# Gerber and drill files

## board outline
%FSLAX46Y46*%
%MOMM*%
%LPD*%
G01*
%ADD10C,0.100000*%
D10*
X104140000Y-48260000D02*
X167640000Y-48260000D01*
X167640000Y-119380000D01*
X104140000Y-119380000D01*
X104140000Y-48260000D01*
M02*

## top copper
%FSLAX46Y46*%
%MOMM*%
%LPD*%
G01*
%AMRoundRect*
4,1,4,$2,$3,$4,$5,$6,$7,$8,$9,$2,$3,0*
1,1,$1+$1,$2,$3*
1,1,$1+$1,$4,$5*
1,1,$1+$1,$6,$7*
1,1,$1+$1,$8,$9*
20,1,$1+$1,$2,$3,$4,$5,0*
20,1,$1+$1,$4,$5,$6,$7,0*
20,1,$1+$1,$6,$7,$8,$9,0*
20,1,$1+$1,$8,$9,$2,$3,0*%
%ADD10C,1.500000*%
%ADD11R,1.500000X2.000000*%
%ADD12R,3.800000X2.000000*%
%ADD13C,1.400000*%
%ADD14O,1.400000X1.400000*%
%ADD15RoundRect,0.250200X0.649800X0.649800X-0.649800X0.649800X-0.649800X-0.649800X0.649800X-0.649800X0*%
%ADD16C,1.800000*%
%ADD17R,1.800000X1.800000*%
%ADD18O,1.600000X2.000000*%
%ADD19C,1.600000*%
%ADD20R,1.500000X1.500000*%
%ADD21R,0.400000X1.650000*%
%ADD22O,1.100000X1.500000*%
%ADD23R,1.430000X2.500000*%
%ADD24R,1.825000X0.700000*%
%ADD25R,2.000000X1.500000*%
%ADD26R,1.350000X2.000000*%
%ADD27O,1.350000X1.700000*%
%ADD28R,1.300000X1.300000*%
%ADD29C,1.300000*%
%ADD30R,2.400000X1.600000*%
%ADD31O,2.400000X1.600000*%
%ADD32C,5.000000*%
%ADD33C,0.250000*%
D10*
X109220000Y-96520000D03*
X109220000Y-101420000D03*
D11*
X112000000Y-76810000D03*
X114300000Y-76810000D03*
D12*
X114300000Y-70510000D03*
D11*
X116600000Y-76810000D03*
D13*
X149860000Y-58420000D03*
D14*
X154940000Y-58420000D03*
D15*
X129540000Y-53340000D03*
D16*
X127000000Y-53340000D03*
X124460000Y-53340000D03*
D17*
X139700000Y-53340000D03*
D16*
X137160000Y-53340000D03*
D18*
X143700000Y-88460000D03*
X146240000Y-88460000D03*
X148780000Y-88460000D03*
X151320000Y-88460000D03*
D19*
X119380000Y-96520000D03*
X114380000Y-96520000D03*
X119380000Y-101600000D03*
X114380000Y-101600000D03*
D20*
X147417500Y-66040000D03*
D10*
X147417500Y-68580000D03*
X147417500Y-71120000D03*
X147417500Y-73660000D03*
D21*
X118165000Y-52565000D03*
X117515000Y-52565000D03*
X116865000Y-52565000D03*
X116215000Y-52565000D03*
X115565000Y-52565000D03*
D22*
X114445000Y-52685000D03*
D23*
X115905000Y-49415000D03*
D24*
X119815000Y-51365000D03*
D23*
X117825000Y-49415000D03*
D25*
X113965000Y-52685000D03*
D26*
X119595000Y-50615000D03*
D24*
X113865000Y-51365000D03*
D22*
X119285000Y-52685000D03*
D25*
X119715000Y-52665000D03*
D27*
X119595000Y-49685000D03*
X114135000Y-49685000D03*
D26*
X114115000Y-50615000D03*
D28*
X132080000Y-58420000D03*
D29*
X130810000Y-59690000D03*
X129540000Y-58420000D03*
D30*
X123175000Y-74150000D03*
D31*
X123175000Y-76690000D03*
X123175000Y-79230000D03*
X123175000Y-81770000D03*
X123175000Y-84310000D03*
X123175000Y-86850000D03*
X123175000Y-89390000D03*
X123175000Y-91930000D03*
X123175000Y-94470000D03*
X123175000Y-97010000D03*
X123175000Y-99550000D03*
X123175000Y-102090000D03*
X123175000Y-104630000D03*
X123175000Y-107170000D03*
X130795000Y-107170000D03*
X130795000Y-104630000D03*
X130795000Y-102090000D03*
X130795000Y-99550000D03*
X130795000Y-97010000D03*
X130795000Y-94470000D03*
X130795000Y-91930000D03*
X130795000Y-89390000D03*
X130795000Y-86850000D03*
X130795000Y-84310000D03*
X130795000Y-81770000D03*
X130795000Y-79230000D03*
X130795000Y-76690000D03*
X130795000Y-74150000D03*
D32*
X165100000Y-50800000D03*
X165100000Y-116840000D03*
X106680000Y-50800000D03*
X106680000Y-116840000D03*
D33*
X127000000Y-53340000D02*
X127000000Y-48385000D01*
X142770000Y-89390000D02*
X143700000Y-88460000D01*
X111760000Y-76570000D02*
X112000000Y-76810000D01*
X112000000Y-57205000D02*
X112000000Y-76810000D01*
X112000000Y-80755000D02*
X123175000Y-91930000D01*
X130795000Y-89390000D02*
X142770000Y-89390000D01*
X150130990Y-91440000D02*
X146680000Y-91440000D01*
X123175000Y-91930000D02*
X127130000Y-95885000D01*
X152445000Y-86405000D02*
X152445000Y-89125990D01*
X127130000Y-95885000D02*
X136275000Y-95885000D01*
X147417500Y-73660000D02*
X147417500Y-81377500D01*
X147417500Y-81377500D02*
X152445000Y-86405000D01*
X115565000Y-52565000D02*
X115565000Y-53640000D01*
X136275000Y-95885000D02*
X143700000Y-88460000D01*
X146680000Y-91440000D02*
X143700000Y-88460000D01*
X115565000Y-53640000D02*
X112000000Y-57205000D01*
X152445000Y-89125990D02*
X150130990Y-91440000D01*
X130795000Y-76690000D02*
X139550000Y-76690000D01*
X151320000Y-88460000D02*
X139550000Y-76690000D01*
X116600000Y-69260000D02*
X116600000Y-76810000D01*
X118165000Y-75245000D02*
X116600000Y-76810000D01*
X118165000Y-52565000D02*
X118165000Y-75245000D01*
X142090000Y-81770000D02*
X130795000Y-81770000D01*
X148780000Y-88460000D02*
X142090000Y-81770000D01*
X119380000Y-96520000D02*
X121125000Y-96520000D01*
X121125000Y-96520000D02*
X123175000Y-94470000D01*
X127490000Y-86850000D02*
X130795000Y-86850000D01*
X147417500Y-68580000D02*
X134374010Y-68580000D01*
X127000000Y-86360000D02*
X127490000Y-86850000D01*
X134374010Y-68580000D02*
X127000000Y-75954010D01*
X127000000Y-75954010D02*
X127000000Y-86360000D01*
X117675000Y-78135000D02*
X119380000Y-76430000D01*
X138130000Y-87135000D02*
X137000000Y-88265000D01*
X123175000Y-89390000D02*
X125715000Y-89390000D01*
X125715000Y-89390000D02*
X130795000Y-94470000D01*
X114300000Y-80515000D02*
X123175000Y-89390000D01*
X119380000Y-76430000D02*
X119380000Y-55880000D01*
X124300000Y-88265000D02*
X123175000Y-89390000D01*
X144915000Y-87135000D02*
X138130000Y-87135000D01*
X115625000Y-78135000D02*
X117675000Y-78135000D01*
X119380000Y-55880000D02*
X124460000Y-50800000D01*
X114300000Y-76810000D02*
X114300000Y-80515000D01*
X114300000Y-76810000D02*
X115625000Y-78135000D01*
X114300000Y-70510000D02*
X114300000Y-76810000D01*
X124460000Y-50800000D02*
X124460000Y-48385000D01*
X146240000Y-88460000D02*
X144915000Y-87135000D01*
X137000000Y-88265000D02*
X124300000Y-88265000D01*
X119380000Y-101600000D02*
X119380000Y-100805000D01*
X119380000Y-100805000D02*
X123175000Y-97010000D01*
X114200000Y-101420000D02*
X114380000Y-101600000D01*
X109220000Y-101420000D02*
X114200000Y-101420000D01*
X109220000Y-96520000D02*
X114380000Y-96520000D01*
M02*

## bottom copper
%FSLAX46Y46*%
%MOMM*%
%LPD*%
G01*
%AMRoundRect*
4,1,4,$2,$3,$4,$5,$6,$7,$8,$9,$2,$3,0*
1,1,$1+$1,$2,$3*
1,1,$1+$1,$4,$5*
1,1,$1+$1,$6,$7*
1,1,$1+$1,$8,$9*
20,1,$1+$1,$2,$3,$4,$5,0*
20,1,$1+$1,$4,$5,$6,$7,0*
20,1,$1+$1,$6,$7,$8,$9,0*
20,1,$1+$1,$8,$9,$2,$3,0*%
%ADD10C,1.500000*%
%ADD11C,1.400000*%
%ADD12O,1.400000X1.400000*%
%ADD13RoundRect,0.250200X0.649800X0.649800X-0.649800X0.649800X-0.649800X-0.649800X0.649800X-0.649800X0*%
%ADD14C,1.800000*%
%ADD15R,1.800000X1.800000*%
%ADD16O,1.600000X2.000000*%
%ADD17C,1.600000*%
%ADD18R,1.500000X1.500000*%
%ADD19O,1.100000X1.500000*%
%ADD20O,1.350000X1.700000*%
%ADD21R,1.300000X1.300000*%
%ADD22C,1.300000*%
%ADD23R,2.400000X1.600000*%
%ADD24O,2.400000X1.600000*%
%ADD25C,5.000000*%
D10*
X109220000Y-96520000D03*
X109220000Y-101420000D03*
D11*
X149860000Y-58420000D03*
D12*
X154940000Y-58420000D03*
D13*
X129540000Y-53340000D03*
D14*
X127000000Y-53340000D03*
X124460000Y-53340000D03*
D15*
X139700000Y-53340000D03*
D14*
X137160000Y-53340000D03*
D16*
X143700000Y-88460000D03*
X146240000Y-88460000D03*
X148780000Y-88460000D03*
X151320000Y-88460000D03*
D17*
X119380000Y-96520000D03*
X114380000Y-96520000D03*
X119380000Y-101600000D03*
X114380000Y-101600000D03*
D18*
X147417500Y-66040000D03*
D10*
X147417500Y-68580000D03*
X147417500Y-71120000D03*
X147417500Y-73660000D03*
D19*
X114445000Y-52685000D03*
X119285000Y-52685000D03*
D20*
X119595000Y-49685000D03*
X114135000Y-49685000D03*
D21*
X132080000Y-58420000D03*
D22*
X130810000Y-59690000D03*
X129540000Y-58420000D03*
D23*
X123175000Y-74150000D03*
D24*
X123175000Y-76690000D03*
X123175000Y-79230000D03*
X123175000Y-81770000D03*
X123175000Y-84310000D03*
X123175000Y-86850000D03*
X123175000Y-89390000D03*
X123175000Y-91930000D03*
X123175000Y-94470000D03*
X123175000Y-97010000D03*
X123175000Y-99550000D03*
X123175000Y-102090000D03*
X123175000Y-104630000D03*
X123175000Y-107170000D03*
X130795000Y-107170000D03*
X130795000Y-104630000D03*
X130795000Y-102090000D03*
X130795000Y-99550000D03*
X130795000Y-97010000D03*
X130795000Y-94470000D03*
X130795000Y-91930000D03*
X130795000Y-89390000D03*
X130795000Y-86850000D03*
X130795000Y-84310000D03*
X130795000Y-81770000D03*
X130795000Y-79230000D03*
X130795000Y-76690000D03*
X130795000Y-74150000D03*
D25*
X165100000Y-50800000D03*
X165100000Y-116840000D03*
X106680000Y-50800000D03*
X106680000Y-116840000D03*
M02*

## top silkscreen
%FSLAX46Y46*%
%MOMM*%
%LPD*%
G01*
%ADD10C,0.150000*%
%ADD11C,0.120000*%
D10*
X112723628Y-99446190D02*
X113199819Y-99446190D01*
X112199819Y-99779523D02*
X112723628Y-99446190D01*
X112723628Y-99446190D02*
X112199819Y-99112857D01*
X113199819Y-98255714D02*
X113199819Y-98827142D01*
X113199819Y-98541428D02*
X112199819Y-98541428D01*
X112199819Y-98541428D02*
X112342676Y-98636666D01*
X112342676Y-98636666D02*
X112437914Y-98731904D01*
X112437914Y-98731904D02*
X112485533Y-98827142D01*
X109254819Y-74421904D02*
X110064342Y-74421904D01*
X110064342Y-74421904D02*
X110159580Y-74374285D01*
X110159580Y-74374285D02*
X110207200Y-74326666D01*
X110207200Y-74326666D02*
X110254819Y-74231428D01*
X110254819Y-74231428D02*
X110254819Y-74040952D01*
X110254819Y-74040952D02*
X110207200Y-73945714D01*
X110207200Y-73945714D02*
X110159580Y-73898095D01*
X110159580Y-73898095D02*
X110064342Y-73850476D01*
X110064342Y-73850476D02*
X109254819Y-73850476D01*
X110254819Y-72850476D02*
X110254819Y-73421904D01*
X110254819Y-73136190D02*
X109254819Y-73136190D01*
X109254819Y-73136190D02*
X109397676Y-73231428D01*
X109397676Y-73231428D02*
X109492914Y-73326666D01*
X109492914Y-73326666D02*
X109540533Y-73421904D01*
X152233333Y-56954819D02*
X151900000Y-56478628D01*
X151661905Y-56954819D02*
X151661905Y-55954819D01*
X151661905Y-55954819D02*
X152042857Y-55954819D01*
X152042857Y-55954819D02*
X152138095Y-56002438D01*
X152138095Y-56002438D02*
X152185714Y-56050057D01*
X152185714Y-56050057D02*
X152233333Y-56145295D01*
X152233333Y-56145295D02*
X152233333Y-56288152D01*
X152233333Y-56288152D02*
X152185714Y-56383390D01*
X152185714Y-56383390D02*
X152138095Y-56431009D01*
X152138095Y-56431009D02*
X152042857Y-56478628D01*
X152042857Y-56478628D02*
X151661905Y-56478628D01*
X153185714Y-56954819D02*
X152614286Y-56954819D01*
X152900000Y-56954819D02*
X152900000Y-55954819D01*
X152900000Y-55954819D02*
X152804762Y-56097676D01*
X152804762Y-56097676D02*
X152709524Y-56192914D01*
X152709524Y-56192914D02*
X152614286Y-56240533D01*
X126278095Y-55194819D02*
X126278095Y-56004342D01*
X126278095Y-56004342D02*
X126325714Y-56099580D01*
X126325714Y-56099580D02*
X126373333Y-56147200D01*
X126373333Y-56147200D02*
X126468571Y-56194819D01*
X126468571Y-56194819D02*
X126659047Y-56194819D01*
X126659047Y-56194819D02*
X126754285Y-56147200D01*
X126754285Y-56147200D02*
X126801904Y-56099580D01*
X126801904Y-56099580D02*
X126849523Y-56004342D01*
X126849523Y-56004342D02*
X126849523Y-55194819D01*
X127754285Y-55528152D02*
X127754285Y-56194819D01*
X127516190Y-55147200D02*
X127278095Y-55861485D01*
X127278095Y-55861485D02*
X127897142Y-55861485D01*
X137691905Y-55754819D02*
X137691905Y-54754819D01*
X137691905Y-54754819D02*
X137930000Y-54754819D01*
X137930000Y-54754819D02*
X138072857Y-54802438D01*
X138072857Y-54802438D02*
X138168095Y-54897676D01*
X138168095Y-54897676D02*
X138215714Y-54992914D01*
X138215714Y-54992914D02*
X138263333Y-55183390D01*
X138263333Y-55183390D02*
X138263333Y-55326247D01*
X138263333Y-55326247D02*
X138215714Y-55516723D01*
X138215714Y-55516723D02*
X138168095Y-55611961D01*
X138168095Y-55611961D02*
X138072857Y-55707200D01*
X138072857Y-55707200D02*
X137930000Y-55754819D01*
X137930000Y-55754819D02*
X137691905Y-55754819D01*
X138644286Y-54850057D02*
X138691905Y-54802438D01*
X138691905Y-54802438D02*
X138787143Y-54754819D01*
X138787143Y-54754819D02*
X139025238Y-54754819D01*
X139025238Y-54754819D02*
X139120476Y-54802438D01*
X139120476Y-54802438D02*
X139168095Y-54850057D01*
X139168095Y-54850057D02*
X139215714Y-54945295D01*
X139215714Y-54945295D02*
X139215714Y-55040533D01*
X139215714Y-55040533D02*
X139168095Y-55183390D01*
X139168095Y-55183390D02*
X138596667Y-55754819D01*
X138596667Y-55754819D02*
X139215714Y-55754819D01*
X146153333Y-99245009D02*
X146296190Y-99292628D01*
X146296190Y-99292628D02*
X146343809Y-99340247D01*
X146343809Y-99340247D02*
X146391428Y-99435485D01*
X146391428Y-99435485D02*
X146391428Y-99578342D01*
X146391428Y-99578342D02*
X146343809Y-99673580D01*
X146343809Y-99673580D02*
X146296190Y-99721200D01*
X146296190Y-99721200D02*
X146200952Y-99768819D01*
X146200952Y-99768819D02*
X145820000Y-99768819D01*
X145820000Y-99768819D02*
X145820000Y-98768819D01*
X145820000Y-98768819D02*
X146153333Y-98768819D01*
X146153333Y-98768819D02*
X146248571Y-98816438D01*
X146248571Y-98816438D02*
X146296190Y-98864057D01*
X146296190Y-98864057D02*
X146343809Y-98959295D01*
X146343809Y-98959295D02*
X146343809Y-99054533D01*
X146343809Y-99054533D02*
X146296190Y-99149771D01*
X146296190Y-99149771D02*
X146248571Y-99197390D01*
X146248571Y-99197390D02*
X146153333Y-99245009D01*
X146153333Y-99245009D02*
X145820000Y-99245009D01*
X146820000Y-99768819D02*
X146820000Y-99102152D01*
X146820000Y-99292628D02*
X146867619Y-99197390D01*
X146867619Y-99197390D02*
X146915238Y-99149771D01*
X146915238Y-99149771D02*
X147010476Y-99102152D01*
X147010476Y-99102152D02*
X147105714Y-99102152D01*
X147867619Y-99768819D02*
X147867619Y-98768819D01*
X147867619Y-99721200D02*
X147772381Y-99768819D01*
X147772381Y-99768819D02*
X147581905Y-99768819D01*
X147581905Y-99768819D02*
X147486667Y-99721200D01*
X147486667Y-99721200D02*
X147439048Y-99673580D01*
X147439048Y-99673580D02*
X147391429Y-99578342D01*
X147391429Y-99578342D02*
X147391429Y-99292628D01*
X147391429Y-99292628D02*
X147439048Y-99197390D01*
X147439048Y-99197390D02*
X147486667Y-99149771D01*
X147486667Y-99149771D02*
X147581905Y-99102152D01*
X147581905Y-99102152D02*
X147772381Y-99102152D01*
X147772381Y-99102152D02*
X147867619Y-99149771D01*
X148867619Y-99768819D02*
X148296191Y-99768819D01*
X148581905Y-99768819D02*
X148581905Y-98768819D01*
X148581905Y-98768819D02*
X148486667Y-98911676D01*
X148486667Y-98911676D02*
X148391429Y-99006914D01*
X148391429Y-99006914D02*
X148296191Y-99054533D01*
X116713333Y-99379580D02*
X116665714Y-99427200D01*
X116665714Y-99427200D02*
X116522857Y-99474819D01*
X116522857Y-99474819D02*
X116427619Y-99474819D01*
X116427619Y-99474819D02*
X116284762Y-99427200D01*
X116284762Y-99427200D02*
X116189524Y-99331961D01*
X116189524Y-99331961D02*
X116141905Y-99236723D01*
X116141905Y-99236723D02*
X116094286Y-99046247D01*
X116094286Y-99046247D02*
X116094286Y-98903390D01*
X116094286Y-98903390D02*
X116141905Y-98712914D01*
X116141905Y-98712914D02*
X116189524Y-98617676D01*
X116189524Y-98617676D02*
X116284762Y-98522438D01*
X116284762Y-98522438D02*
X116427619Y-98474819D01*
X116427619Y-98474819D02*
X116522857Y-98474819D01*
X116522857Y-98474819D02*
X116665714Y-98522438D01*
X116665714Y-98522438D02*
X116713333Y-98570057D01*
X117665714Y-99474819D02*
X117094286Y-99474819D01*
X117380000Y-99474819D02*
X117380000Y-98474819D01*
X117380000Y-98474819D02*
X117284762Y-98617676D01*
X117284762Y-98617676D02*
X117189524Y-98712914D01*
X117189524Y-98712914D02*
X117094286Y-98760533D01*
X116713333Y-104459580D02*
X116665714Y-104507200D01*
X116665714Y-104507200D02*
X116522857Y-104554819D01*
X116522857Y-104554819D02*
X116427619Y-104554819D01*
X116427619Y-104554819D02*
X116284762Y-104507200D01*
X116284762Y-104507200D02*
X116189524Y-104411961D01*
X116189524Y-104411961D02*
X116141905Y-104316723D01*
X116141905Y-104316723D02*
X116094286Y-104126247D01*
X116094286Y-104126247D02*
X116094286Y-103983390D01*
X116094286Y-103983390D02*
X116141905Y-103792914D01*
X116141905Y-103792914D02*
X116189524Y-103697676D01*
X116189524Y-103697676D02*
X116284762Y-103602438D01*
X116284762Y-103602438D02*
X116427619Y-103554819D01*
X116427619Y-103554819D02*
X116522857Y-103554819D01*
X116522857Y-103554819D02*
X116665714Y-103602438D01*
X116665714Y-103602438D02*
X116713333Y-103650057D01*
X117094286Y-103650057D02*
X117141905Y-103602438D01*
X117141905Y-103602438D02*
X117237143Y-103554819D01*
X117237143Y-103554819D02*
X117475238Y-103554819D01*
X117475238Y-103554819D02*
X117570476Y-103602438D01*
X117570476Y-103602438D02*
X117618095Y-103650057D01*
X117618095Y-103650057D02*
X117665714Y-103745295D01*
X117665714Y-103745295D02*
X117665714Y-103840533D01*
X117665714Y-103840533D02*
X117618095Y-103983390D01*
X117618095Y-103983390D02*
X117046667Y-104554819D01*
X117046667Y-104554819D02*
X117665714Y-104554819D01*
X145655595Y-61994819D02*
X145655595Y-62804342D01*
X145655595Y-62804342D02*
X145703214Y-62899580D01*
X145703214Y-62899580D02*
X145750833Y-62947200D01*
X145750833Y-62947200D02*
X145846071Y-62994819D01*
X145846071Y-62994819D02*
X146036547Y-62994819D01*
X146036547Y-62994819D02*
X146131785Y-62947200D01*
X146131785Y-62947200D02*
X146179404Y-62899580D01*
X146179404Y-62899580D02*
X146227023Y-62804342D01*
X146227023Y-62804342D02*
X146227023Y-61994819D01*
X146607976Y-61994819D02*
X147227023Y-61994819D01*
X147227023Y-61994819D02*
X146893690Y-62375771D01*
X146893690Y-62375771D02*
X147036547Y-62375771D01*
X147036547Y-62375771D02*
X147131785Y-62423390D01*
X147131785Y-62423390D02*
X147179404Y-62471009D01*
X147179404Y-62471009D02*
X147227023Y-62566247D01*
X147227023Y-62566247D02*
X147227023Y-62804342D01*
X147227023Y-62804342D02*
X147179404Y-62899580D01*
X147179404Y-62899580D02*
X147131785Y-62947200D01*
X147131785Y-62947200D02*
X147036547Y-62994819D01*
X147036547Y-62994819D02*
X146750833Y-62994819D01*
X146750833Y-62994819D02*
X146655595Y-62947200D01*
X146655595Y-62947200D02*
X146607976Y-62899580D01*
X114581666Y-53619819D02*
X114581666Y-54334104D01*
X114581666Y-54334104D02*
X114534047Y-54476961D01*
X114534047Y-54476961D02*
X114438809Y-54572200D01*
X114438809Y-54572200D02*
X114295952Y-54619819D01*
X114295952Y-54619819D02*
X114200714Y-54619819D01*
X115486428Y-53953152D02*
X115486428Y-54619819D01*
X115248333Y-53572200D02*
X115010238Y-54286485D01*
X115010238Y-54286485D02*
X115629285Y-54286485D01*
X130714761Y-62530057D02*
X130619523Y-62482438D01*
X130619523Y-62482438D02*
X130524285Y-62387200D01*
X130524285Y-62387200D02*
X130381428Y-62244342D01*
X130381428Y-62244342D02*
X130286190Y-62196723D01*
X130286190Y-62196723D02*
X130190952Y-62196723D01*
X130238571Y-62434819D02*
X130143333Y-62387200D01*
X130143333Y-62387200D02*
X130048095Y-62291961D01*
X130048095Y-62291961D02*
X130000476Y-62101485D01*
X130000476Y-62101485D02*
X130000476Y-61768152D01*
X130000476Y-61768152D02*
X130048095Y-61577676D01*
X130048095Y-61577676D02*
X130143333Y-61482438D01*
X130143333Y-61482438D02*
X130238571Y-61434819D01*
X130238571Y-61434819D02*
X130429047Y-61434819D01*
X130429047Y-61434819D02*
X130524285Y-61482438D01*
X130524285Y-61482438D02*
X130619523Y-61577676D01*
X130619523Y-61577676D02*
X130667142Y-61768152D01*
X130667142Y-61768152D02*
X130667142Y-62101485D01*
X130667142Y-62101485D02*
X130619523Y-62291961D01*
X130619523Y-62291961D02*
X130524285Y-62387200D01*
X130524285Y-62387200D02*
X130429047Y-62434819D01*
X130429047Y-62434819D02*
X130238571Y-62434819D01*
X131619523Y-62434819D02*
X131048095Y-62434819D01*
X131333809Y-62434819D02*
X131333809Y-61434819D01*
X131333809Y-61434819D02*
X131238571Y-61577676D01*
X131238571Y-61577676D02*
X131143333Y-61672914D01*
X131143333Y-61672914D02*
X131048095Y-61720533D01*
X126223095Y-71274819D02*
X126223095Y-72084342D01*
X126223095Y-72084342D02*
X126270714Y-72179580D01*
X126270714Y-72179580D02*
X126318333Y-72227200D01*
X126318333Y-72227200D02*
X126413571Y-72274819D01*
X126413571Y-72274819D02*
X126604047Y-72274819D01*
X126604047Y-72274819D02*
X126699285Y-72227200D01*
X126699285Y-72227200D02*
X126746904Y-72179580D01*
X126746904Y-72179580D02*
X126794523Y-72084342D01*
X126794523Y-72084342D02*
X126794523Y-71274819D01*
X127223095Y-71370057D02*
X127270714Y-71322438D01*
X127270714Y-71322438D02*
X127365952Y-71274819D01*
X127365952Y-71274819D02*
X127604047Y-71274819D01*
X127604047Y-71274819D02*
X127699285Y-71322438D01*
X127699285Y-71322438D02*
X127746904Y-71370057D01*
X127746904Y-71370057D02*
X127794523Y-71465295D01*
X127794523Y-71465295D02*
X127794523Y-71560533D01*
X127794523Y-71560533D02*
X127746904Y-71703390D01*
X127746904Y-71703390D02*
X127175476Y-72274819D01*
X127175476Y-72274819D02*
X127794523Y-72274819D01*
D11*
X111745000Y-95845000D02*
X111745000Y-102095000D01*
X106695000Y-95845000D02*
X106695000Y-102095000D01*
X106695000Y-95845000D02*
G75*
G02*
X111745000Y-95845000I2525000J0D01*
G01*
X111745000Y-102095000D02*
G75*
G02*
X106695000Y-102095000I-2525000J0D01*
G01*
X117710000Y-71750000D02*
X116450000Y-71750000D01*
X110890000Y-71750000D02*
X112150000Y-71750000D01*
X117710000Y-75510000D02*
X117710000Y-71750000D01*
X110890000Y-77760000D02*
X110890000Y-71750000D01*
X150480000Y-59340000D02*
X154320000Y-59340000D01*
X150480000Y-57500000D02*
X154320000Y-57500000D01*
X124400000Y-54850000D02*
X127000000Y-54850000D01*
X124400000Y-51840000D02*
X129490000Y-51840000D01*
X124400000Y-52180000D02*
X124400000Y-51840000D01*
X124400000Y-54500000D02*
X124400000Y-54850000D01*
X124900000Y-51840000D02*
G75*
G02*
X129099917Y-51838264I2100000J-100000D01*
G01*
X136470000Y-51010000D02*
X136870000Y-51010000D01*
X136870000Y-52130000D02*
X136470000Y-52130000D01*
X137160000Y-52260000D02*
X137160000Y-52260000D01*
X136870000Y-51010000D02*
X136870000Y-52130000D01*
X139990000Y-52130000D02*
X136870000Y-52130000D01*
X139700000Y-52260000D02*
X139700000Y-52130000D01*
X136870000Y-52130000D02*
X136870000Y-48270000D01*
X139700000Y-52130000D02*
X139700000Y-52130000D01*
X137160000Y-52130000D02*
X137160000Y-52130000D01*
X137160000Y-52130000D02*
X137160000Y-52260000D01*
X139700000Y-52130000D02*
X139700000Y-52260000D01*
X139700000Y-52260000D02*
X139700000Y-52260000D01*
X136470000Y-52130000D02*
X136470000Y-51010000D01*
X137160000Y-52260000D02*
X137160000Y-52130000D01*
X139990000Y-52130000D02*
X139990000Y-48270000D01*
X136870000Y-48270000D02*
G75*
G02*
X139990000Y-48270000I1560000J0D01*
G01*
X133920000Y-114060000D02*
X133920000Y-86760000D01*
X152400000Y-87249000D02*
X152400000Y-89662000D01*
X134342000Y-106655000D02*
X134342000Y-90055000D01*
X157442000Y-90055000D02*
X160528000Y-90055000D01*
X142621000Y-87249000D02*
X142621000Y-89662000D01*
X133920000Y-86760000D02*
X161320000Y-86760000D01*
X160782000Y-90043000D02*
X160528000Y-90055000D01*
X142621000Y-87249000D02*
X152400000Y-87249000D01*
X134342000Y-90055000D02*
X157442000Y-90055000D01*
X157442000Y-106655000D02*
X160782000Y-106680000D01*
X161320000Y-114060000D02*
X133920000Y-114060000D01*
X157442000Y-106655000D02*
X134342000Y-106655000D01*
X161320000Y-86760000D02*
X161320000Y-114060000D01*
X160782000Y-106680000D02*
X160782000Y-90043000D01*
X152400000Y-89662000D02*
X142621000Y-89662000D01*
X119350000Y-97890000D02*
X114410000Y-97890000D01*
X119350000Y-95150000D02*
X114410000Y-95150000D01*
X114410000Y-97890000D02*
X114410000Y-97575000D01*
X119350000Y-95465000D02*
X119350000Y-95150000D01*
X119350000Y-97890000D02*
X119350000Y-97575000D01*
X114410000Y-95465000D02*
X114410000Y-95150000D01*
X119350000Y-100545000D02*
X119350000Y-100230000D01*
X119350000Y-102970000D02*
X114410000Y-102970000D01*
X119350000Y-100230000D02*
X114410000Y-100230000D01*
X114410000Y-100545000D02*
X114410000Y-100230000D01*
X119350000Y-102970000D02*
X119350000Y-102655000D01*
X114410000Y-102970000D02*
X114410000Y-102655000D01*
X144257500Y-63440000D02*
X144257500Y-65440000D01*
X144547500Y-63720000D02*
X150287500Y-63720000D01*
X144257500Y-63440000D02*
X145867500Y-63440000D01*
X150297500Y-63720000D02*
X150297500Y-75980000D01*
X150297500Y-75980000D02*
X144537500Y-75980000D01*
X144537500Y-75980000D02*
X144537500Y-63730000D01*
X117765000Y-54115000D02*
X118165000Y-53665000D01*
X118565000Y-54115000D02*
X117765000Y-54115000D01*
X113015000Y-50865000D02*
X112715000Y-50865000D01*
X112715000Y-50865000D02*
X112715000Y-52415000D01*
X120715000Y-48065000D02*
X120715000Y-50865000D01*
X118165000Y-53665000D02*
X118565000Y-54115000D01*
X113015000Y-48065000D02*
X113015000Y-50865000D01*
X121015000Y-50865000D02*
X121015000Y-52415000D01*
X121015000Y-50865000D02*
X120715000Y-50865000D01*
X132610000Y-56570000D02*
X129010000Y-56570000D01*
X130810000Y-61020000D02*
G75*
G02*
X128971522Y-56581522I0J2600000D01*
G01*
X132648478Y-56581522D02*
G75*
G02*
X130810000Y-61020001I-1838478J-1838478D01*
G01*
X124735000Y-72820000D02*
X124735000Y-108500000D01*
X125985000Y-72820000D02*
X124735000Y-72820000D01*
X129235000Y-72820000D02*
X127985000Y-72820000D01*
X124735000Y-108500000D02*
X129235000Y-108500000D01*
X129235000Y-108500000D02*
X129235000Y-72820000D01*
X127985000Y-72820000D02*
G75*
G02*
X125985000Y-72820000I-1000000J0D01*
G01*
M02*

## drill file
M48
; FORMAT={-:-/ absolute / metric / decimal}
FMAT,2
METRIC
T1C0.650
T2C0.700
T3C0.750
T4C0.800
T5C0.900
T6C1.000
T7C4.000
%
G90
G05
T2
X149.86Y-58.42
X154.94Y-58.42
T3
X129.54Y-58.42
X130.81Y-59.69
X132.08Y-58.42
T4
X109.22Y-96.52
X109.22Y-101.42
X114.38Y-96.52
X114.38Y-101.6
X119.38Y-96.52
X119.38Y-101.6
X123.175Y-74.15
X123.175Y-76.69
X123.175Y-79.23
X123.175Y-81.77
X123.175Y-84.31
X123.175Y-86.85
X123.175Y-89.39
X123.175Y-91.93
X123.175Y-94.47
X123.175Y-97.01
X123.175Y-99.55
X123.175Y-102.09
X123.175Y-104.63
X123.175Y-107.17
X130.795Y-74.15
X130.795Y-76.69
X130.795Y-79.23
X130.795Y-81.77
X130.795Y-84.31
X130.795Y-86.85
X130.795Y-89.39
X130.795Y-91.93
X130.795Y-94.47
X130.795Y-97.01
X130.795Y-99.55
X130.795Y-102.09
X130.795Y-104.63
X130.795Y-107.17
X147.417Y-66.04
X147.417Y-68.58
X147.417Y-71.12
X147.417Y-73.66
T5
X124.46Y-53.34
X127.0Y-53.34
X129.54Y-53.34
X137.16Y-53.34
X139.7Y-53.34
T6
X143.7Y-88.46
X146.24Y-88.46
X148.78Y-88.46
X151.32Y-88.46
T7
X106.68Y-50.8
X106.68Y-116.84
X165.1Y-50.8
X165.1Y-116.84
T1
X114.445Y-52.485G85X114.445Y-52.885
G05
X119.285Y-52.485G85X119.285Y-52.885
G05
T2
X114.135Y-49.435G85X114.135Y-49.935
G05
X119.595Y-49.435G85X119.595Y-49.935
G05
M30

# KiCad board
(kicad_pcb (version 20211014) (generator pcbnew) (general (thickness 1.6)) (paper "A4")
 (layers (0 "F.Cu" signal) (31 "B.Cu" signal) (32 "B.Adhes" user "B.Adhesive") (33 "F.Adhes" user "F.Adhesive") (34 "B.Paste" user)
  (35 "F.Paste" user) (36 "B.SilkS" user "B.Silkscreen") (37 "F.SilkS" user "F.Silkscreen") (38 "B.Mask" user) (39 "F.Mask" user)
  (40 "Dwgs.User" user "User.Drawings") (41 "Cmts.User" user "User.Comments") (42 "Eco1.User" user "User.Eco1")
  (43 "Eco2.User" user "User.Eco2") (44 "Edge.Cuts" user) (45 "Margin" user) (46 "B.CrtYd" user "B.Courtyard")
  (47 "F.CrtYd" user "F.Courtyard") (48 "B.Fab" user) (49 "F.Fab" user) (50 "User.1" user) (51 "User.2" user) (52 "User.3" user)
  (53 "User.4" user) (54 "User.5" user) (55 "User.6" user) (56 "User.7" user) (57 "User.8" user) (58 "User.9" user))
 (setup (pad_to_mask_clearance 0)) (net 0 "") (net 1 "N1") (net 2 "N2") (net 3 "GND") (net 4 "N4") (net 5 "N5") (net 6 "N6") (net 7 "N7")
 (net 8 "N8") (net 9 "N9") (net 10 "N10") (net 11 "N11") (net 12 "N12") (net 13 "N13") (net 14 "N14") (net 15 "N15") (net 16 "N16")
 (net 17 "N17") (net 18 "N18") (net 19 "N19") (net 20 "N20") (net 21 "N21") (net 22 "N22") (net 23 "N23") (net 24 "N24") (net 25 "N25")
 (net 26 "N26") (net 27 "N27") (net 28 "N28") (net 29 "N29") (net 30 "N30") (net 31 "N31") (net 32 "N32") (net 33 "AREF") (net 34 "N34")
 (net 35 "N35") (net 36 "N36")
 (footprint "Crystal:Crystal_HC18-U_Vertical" (layer "F.Cu") (at 109.22 96.52 -90)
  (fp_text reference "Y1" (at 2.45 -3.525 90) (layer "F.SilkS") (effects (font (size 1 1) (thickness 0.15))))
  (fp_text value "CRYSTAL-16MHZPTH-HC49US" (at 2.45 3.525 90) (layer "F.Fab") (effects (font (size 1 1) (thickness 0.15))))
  (fp_line (start -0.675 -2.525) (end 5.575 -2.525) (layer "F.SilkS") (width 0.12))
  (fp_line (start -0.675 2.525) (end 5.575 2.525) (layer "F.SilkS") (width 0.12))
  (fp_arc (start -0.675 2.525) (mid -3.2 0) (end -0.675 -2.525) (layer "F.SilkS") (width 0.12))
  (fp_arc (start 5.575 -2.525) (mid 8.1 0) (end 5.575 2.525) (layer "F.SilkS") (width 0.12))
  (pad "1" thru_hole circle (at 0 0 270) (size 1.5 1.5) (drill 0.8) (layers *.Cu *.Mask) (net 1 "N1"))
  (pad "2" thru_hole circle (at 4.9 0 270) (size 1.5 1.5) (drill 0.8) (layers *.Cu *.Mask) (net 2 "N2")))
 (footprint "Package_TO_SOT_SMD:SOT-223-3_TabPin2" (layer "F.Cu") (at 114.3 73.66 90)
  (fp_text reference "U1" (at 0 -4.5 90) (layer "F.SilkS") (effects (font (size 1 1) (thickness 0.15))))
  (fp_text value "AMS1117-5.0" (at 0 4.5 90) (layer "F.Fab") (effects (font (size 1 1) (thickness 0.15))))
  (fp_line (start 1.91 3.41) (end 1.91 2.15) (layer "F.SilkS") (width 0.12))
  (fp_line (start 1.91 -3.41) (end 1.91 -2.15) (layer "F.SilkS") (width 0.12))
  (fp_line (start -1.85 3.41) (end 1.91 3.41) (layer "F.SilkS") (width 0.12))
  (fp_line (start -4.1 -3.41) (end 1.91 -3.41) (layer "F.SilkS") (width 0.12))
  (pad "1" smd rect (at -3.15 -2.3 90) (size 2 1.5) (layers "F.Cu" "F.Paste" "F.Mask") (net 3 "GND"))
  (pad "2" smd rect (at -3.15 0 90) (size 2 1.5) (layers "F.Cu" "F.Paste" "F.Mask") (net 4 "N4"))
  (pad "2" smd rect (at 3.15 0 90) (size 2 3.8) (layers "F.Cu" "F.Paste" "F.Mask") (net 4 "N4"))
  (pad "3" smd rect (at -3.15 2.3 90) (size 2 1.5) (layers "F.Cu" "F.Paste" "F.Mask") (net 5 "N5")))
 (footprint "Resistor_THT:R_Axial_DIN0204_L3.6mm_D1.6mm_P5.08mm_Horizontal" (layer "F.Cu") (at 149.86 58.42)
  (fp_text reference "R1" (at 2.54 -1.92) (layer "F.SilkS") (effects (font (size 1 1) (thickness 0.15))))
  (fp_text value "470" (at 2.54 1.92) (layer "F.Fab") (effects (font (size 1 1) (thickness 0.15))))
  (fp_line (start 0.62 0.92) (end 4.46 0.92) (layer "F.SilkS") (width 0.12))
  (fp_line (start 0.62 -0.92) (end 4.46 -0.92) (layer "F.SilkS") (width 0.12))
  (pad "1" thru_hole circle (at 0 0) (size 1.4 1.4) (drill 0.7) (layers *.Cu *.Mask) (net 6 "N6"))
  (pad "2" thru_hole oval (at 5.08 0) (size 1.4 1.4) (drill 0.7) (layers *.Cu *.Mask) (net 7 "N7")))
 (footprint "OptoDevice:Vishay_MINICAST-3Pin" (layer "F.Cu") (at 129.54 53.34 180)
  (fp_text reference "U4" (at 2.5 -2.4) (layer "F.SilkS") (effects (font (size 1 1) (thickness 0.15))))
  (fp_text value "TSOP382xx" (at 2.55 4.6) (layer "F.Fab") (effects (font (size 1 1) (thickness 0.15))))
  (fp_line (start 5.14 -1.51) (end 2.54 -1.51) (layer "F.SilkS") (width 0.12))
  (fp_line (start 5.14 1.5) (end 0.05 1.5) (layer "F.SilkS") (width 0.12))
  (fp_line (start 5.14 1.16) (end 5.14 1.5) (layer "F.SilkS") (width 0.12))
  (fp_line (start 5.14 -1.16) (end 5.14 -1.51) (layer "F.SilkS") (width 0.12))
  (fp_arc (start 4.64 1.5) (mid 2.540869 3.502379) (end 0.440083 1.501736) (layer "F.SilkS") (width 0.12))
  (pad "1" thru_hole roundrect (at 0 0 180) (size 1.8 1.8) (drill 0.9) (layers *.Cu *.Mask) (roundrect_rratio 0.139) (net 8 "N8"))
  (pad "2" thru_hole circle (at 2.54 0 180) (size 1.8 1.8) (drill 0.9) (layers *.Cu *.Mask) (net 3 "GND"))
  (pad "3" thru_hole circle (at 5.08 0 180) (size 1.8 1.8) (drill 0.9) (layers *.Cu *.Mask) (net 4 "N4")))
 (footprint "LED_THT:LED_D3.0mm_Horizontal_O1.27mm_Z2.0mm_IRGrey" (layer "F.Cu") (at 139.7 53.34 180)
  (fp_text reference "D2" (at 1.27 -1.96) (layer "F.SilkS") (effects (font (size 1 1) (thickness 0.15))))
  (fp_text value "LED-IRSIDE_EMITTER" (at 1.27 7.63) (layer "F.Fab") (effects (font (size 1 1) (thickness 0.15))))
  (fp_line (start 3.23 2.33) (end 2.83 2.33) (layer "F.SilkS") (width 0.12))
  (fp_line (start 2.83 1.21) (end 3.23 1.21) (layer "F.SilkS") (width 0.12))
  (fp_line (start 2.54 1.08) (end 2.54 1.08) (layer "F.SilkS") (width 0.12))
  (fp_line (start 2.83 2.33) (end 2.83 1.21) (layer "F.SilkS") (width 0.12))
  (fp_line (start -0.29 1.21) (end 2.83 1.21) (layer "F.SilkS") (width 0.12))
  (fp_line (start 0 1.08) (end 0 1.21) (layer "F.SilkS") (width 0.12))
  (fp_line (start 2.83 1.21) (end 2.83 5.07) (layer "F.SilkS") (width 0.12))
  (fp_line (start 0 1.21) (end 0 1.21) (layer "F.SilkS") (width 0.12))
  (fp_line (start 2.54 1.21) (end 2.54 1.21) (layer "F.SilkS") (width 0.12))
  (fp_line (start 2.54 1.21) (end 2.54 1.08) (layer "F.SilkS") (width 0.12))
  (fp_line (start 0 1.21) (end 0 1.08) (layer "F.SilkS") (width 0.12))
  (fp_line (start 0 1.08) (end 0 1.08) (layer "F.SilkS") (width 0.12))
  (fp_line (start 3.23 1.21) (end 3.23 2.33) (layer "F.SilkS") (width 0.12))
  (fp_line (start 2.54 1.08) (end 2.54 1.21) (layer "F.SilkS") (width 0.12))
  (fp_line (start -0.29 1.21) (end -0.29 5.07) (layer "F.SilkS") (width 0.12))
  (fp_arc (start 2.83 5.07) (mid 1.27 6.63) (end -0.29 5.07) (layer "F.SilkS") (width 0.12))
  (pad "1" thru_hole rect (at 0 0 180) (size 1.8 1.8) (drill 0.9) (layers *.Cu *.Mask))
  (pad "2" thru_hole circle (at 2.54 0 180) (size 1.8 1.8) (drill 0.9) (layers *.Cu *.Mask)))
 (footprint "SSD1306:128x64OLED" (layer "F.Cu") (at 147.32 99.06)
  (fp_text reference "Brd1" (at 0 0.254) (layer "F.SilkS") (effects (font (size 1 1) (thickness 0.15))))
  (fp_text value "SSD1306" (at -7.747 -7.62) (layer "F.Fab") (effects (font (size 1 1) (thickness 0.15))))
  (fp_line (start -13.4 15) (end -13.4 -12.3) (layer "F.SilkS") (width 0.12))
  (fp_line (start 5.08 -11.811) (end 5.08 -9.398) (layer "F.SilkS") (width 0.12))
  (fp_line (start -12.978 7.595) (end -12.978 -9.005) (layer "F.SilkS") (width 0.12))
  (fp_line (start 10.122 -9.005) (end 13.208 -9.005) (layer "F.SilkS") (width 0.12))
  (fp_line (start -4.699 -11.811) (end -4.699 -9.398) (layer "F.SilkS") (width 0.12))
  (fp_line (start -13.4 -12.3) (end 14 -12.3) (layer "F.SilkS") (width 0.12))
  (fp_line (start 13.462 -9.017) (end 13.208 -9.005) (layer "F.SilkS") (width 0.12))
  (fp_line (start -4.699 -11.811) (end 5.08 -11.811) (layer "F.SilkS") (width 0.12))
  (fp_line (start -12.978 -9.005) (end 10.122 -9.005) (layer "F.SilkS") (width 0.12))
  (fp_line (start 10.122 7.595) (end 13.462 7.62) (layer "F.SilkS") (width 0.12))
  (fp_line (start 14 15) (end -13.4 15) (layer "F.SilkS") (width 0.12))
  (fp_line (start 10.122 7.595) (end -12.978 7.595) (layer "F.SilkS") (width 0.12))
  (fp_line (start 14 -12.3) (end 14 15) (layer "F.SilkS") (width 0.12))
  (fp_line (start 13.462 7.62) (end 13.462 -9.017) (layer "F.SilkS") (width 0.12))
  (fp_line (start 5.08 -9.398) (end -4.699 -9.398) (layer "F.SilkS") (width 0.12))
  (pad "1" thru_hole oval locked (at -3.62 -10.6 90) (size 2 1.6) (drill 1) (layers *.Cu *.Mask) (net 3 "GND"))
  (pad "2" thru_hole oval locked (at -1.08 -10.6 90) (size 2 1.6) (drill 1) (layers *.Cu *.Mask) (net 4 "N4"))
  (pad "3" thru_hole oval locked (at 1.46 -10.6 90) (size 2 1.6) (drill 1) (layers *.Cu *.Mask) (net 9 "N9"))
  (pad "4" thru_hole oval locked (at 4 -10.6 90) (size 2 1.6) (drill 1) (layers *.Cu *.Mask) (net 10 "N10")))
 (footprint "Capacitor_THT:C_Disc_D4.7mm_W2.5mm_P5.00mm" (layer "F.Cu") (at 119.38 96.52 180)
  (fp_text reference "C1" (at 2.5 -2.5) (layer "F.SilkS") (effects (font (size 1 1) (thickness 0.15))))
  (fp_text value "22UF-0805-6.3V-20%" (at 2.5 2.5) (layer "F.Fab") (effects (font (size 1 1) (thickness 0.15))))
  (fp_line (start 0.03 -1.37) (end 4.97 -1.37) (layer "F.SilkS") (width 0.12))
  (fp_line (start 0.03 1.37) (end 4.97 1.37) (layer "F.SilkS") (width 0.12))
  (fp_line (start 4.97 -1.37) (end 4.97 -1.055) (layer "F.SilkS") (width 0.12))
  (fp_line (start 0.03 1.055) (end 0.03 1.37) (layer "F.SilkS") (width 0.12))
  (fp_line (start 0.03 -1.37) (end 0.03 -1.055) (layer "F.SilkS") (width 0.12))
  (fp_line (start 4.97 1.055) (end 4.97 1.37) (layer "F.SilkS") (width 0.12))
  (pad "1" thru_hole circle (at 0 0 180) (size 1.6 1.6) (drill 0.8) (layers *.Cu *.Mask) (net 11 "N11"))
  (pad "2" thru_hole circle (at 5 0 180) (size 1.6 1.6) (drill 0.8) (layers *.Cu *.Mask) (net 1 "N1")))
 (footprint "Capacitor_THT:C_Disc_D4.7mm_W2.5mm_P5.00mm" (layer "F.Cu") (at 119.38 101.6 180)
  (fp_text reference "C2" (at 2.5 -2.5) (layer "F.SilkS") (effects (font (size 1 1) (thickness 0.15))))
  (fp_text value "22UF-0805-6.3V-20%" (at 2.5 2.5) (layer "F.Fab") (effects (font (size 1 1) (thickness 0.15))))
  (fp_line (start 0.03 1.055) (end 0.03 1.37) (layer "F.SilkS") (width 0.12))
  (fp_line (start 0.03 -1.37) (end 4.97 -1.37) (layer "F.SilkS") (width 0.12))
  (fp_line (start 0.03 1.37) (end 4.97 1.37) (layer "F.SilkS") (width 0.12))
  (fp_line (start 4.97 1.055) (end 4.97 1.37) (layer "F.SilkS") (width 0.12))
  (fp_line (start 0.03 -1.37) (end 0.03 -1.055) (layer "F.SilkS") (width 0.12))
  (fp_line (start 4.97 -1.37) (end 4.97 -1.055) (layer "F.SilkS") (width 0.12))
  (pad "1" thru_hole circle (at 0 0 180) (size 1.6 1.6) (drill 0.8) (layers *.Cu *.Mask) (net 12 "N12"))
  (pad "2" thru_hole circle (at 5 0 180) (size 1.6 1.6) (drill 0.8) (layers *.Cu *.Mask) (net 2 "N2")))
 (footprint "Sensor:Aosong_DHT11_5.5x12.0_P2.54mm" (layer "F.Cu") (at 147.4175 66.04)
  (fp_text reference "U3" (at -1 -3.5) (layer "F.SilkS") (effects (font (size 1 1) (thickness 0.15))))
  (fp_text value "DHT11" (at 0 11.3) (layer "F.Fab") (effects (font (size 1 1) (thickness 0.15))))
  (fp_line (start -3.16 -2.6) (end -3.16 -0.6) (layer "F.SilkS") (width 0.12))
  (fp_line (start -2.87 -2.32) (end 2.87 -2.32) (layer "F.SilkS") (width 0.12))
  (fp_line (start -3.16 -2.6) (end -1.55 -2.6) (layer "F.SilkS") (width 0.12))
  (fp_line (start 2.88 -2.32) (end 2.88 9.94) (layer "F.SilkS") (width 0.12))
  (fp_line (start 2.88 9.94) (end -2.88 9.94) (layer "F.SilkS") (width 0.12))
  (fp_line (start -2.88 9.94) (end -2.88 -2.31) (layer "F.SilkS") (width 0.12))
  (pad "1" thru_hole rect (at 0 0) (size 1.5 1.5) (drill 0.8) (layers *.Cu *.Mask) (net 4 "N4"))
  (pad "2" thru_hole circle (at 0 2.54) (size 1.5 1.5) (drill 0.8) (layers *.Cu *.Mask) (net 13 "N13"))
  (pad "3" thru_hole circle (at 0 5.08) (size 1.5 1.5) (drill 0.8) (layers *.Cu *.Mask) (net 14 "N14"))
  (pad "4" thru_hole circle (at 0 7.62) (size 1.5 1.5) (drill 0.8) (layers *.Cu *.Mask) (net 3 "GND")))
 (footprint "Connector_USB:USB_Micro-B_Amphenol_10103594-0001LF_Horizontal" (layer "F.Cu") (at 116.84 50.8 180)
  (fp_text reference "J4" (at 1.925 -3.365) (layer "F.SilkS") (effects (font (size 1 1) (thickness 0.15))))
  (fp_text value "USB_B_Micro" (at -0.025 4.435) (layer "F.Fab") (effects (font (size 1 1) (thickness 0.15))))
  (fp_line (start -0.925 -3.315) (end -1.325 -2.865) (layer "F.SilkS") (width 0.12))
  (fp_line (start -1.725 -3.315) (end -0.925 -3.315) (layer "F.SilkS") (width 0.12))
  (fp_line (start 3.825 -0.065) (end 4.125 -0.065) (layer "F.SilkS") (width 0.12))
  (fp_line (start 4.125 -0.065) (end 4.125 -1.615) (layer "F.SilkS") (width 0.12))
  (fp_line (start -3.875 2.735) (end -3.875 -0.065) (layer "F.SilkS") (width 0.12))
  (fp_line (start -1.325 -2.865) (end -1.725 -3.315) (layer "F.SilkS") (width 0.12))
  (fp_line (start 3.825 2.735) (end 3.825 -0.065) (layer "F.SilkS") (width 0.12))
  (fp_line (start -4.175 -0.065) (end -4.175 -1.615) (layer "F.SilkS") (width 0.12))
  (fp_line (start -4.175 -0.065) (end -3.875 -0.065) (layer "F.SilkS") (width 0.12))
  (pad "1" smd rect (at -1.325 -1.765 270) (size 1.65 0.4) (layers "F.Cu" "F.Paste" "F.Mask") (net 5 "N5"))
  (pad "2" smd rect (at -0.675 -1.765 270) (size 1.65 0.4) (layers "F.Cu" "F.Paste" "F.Mask") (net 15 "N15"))
  (pad "3" smd rect (at -0.025 -1.765 270) (size 1.65 0.4) (layers "F.Cu" "F.Paste" "F.Mask") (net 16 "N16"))
  (pad "4" smd rect (at 0.625 -1.765 270) (size 1.65 0.4) (layers "F.Cu" "F.Paste" "F.Mask") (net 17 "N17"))
  (pad "5" smd rect (at 1.275 -1.765 270) (size 1.65 0.4) (layers "F.Cu" "F.Paste" "F.Mask") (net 3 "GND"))
  (pad "6" thru_hole oval (at 2.395 -1.885 270) (size 1.5 1.1) (drill oval 1.05 0.65) (layers *.Cu *.Mask) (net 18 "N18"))
  (pad "6" smd rect (at 0.935 1.385 270) (size 2.5 1.43) (layers "F.Cu" "F.Paste" "F.Mask") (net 18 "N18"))
  (pad "6" smd rect (at -2.975 -0.565 180) (size 1.825 0.7) (layers "F.Cu" "F.Paste" "F.Mask") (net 18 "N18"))
  (pad "6" smd rect (at -0.985 1.385 270) (size 2.5 1.43) (layers "F.Cu" "F.Paste" "F.Mask") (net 18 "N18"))
  (pad "6" smd rect (at 2.875 -1.885 180) (size 2 1.5) (layers "F.Cu" "F.Paste" "F.Mask") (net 18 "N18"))
  (pad "6" smd rect (at -2.755 0.185 180) (size 1.35 2) (layers "F.Cu" "F.Paste" "F.Mask") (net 18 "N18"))
  (pad "6" smd rect (at 2.975 -0.565 180) (size 1.825 0.7) (layers "F.Cu" "F.Paste" "F.Mask") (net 18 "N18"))
  (pad "6" thru_hole oval (at -2.445 -1.885 270) (size 1.5 1.1) (drill oval 1.05 0.65) (layers *.Cu *.Mask) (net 18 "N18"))
  (pad "6" smd rect (at -2.875 -1.865 180) (size 2 1.5) (layers "F.Cu" "F.Paste" "F.Mask") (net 18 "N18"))
  (pad "6" thru_hole oval (at -2.755 1.115 270) (size 1.7 1.35) (drill oval 1.2 0.7) (layers *.Cu *.Mask) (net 18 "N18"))
  (pad "6" thru_hole oval (at 2.705 1.115 270) (size 1.7 1.35) (drill oval 1.2 0.7) (layers *.Cu *.Mask) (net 18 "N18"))
  (pad "6" smd rect (at 2.725 0.185 180) (size 1.35 2) (layers "F.Cu" "F.Paste" "F.Mask") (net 18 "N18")))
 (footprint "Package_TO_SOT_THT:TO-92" (layer "F.Cu") (at 132.08 58.42 180)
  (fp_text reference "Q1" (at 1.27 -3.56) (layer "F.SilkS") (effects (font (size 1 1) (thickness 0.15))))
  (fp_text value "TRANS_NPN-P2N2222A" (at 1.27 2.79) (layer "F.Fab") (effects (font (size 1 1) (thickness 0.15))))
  (fp_line (start -0.53 1.85) (end 3.07 1.85) (layer "F.SilkS") (width 0.12))
  (fp_arc (start 1.27 -2.6) (mid 3.672087 -0.994977) (end 3.108478 1.838478) (layer "F.SilkS") (width 0.12))
  (fp_arc (start -0.568478 1.838478) (mid -1.132087 -0.994977) (end 1.27 -2.6) (layer "F.SilkS") (width 0.12))
  (pad "1" thru_hole rect (at 0 0 180) (size 1.3 1.3) (drill 0.75) (layers *.Cu *.Mask) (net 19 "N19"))
  (pad "2" thru_hole circle (at 1.27 -1.27 180) (size 1.3 1.3) (drill 0.75) (layers *.Cu *.Mask) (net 7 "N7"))
  (pad "3" thru_hole circle (at 2.54 0 180) (size 1.3 1.3) (drill 0.75) (layers *.Cu *.Mask) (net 3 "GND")))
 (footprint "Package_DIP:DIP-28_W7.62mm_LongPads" (layer "F.Cu") (at 123.175 74.15)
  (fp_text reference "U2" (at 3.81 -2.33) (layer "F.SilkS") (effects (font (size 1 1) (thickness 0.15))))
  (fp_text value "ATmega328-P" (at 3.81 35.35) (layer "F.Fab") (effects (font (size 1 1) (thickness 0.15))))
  (fp_line (start 1.56 -1.33) (end 1.56 34.35) (layer "F.SilkS") (width 0.12))
  (fp_line (start 2.81 -1.33) (end 1.56 -1.33) (layer "F.SilkS") (width 0.12))
  (fp_line (start 6.06 -1.33) (end 4.81 -1.33) (layer "F.SilkS") (width 0.12))
  (fp_line (start 1.56 34.35) (end 6.06 34.35) (layer "F.SilkS") (width 0.12))
  (fp_line (start 6.06 34.35) (end 6.06 -1.33) (layer "F.SilkS") (width 0.12))
  (fp_arc (start 4.81 -1.33) (mid 3.81 -0.33) (end 2.81 -1.33) (layer "F.SilkS") (width 0.12))
  (pad "1" thru_hole rect (at 0 0) (size 2.4 1.6) (drill 0.8) (layers *.Cu *.Mask) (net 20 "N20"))
  (pad "2" thru_hole oval (at 0 2.54) (size 2.4 1.6) (drill 0.8) (layers *.Cu *.Mask) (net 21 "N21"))
  (pad "3" thru_hole oval (at 0 5.08) (size 2.4 1.6) (drill 0.8) (layers *.Cu *.Mask) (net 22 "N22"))
  (pad "4" thru_hole oval (at 0 7.62) (size 2.4 1.6) (drill 0.8) (layers *.Cu *.Mask) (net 6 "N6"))
  (pad "5" thru_hole oval (at 0 10.16) (size 2.4 1.6) (drill 0.8) (layers *.Cu *.Mask) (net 8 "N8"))
  (pad "6" thru_hole oval (at 0 12.7) (size 2.4 1.6) (drill 0.8) (layers *.Cu *.Mask) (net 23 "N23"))
  (pad "7" thru_hole oval (at 0 15.24) (size 2.4 1.6) (drill 0.8) (layers *.Cu *.Mask) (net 4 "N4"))
  (pad "8" thru_hole oval (at 0 17.78) (size 2.4 1.6) (drill 0.8) (layers *.Cu *.Mask) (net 3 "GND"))
  (pad "9" thru_hole oval (at 0 20.32) (size 2.4 1.6) (drill 0.8) (layers *.Cu *.Mask) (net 11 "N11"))
  (pad "10" thru_hole oval (at 0 22.86) (size 2.4 1.6) (drill 0.8) (layers *.Cu *.Mask) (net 12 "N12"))
  (pad "11" thru_hole oval (at 0 25.4) (size 2.4 1.6) (drill 0.8) (layers *.Cu *.Mask) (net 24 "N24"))
  (pad "12" thru_hole oval (at 0 27.94) (size 2.4 1.6) (drill 0.8) (layers *.Cu *.Mask) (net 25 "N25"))
  (pad "13" thru_hole oval (at 0 30.48) (size 2.4 1.6) (drill 0.8) (layers *.Cu *.Mask) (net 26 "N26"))
  (pad "14" thru_hole oval (at 0 33.02) (size 2.4 1.6) (drill 0.8) (layers *.Cu *.Mask) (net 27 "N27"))
  (pad "15" thru_hole oval (at 7.62 33.02) (size 2.4 1.6) (drill 0.8) (layers *.Cu *.Mask) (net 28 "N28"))
  (pad "16" thru_hole oval (at 7.62 30.48) (size 2.4 1.6) (drill 0.8) (layers *.Cu *.Mask) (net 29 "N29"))
  (pad "17" thru_hole oval (at 7.62 27.94) (size 2.4 1.6) (drill 0.8) (layers *.Cu *.Mask) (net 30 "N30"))
  (pad "18" thru_hole oval (at 7.62 25.4) (size 2.4 1.6) (drill 0.8) (layers *.Cu *.Mask) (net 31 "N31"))
  (pad "19" thru_hole oval (at 7.62 22.86) (size 2.4 1.6) (drill 0.8) (layers *.Cu *.Mask) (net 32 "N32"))
  (pad "20" thru_hole oval (at 7.62 20.32) (size 2.4 1.6) (drill 0.8) (layers *.Cu *.Mask) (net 4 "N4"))
  (pad "21" thru_hole oval (at 7.62 17.78) (size 2.4 1.6) (drill 0.8) (layers *.Cu *.Mask) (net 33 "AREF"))
  (pad "22" thru_hole oval (at 7.62 15.24) (size 2.4 1.6) (drill 0.8) (layers *.Cu *.Mask) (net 3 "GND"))
  (pad "23" thru_hole oval (at 7.62 12.7) (size 2.4 1.6) (drill 0.8) (layers *.Cu *.Mask) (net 13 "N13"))
  (pad "24" thru_hole oval (at 7.62 10.16) (size 2.4 1.6) (drill 0.8) (layers *.Cu *.Mask) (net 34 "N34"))
  (pad "25" thru_hole oval (at 7.62 7.62) (size 2.4 1.6) (drill 0.8) (layers *.Cu *.Mask) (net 9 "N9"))
  (pad "26" thru_hole oval (at 7.62 5.08) (size 2.4 1.6) (drill 0.8) (layers *.Cu *.Mask) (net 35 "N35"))
  (pad "27" thru_hole oval (at 7.62 2.54) (size 2.4 1.6) (drill 0.8) (layers *.Cu *.Mask) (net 10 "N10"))
  (pad "28" thru_hole oval (at 7.62 0) (size 2.4 1.6) (drill 0.8) (layers *.Cu *.Mask) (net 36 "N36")))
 (gr_rect (start 104.14 48.26) (end 167.64 119.38) (layer "Edge.Cuts") (width 0.1) (fill none))
 (via (at 165.1 50.8) (size 5) (drill 4) (layers "F.Cu" "B.Cu") (free) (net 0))
 (via (at 165.1 116.84) (size 5) (drill 4) (layers "F.Cu" "B.Cu") (free) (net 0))
 (via (at 106.68 50.8) (size 5) (drill 4) (layers "F.Cu" "B.Cu") (free) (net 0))
 (via (at 106.68 116.84) (size 5) (drill 4) (layers "F.Cu" "B.Cu") (free) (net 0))
 (segment (start 127 53.34) (end 127 48.385) (width 0.25) (layer "F.Cu") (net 3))
 (segment (start 142.77 89.39) (end 143.7 88.46) (width 0.25) (layer "F.Cu") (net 3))
 (segment (start 111.76 76.57) (end 112 76.81) (width 0.25) (layer "F.Cu") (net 3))
 (segment (start 112 57.205) (end 112 76.81) (width 0.25) (layer "F.Cu") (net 3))
 (segment (start 112 80.755) (end 123.175 91.93) (width 0.25) (layer "F.Cu") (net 3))
 (segment (start 130.795 89.39) (end 142.77 89.39) (width 0.25) (layer "F.Cu") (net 3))
 (segment (start 150.13099 91.44) (end 146.68 91.44) (width 0.25) (layer "F.Cu") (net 3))
 (segment (start 123.175 91.93) (end 127.13 95.885) (width 0.25) (layer "F.Cu") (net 3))
 (segment (start 152.445 86.405) (end 152.445 89.12599) (width 0.25) (layer "F.Cu") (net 3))
 (segment (start 127.13 95.885) (end 136.275 95.885) (width 0.25) (layer "F.Cu") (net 3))
 (segment (start 147.4175 73.66) (end 147.4175 81.3775) (width 0.25) (layer "F.Cu") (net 3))
 (segment (start 147.4175 81.3775) (end 152.445 86.405) (width 0.25) (layer "F.Cu") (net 3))
 (segment (start 115.565 52.565) (end 115.565 53.64) (width 0.25) (layer "F.Cu") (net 3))
 (segment (start 136.275 95.885) (end 143.7 88.46) (width 0.25) (layer "F.Cu") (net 3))
 (segment (start 146.68 91.44) (end 143.7 88.46) (width 0.25) (layer "F.Cu") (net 3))
 (segment (start 115.565 53.64) (end 112 57.205) (width 0.25) (layer "F.Cu") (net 3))
 (segment (start 152.445 89.12599) (end 150.13099 91.44) (width 0.25) (layer "F.Cu") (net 3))
 (segment (start 130.795 76.69) (end 139.55 76.69) (width 0.25) (layer "F.Cu") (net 10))
 (segment (start 151.32 88.46) (end 139.55 76.69) (width 0.25) (layer "F.Cu") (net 10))
 (segment (start 116.6 69.26) (end 116.6 76.81) (width 0.25) (layer "F.Cu") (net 5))
 (segment (start 118.165 75.245) (end 116.6 76.81) (width 0.25) (layer "F.Cu") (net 5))
 (segment (start 118.165 52.565) (end 118.165 75.245) (width 0.25) (layer "F.Cu") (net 5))
 (segment (start 142.09 81.77) (end 130.795 81.77) (width 0.25) (layer "F.Cu") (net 9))
 (segment (start 148.78 88.46) (end 142.09 81.77) (width 0.25) (layer "F.Cu") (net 9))
 (segment (start 119.38 96.52) (end 121.125 96.52) (width 0.25) (layer "F.Cu") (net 11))
 (segment (start 121.125 96.52) (end 123.175 94.47) (width 0.25) (layer "F.Cu") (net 11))
 (segment (start 127.49 86.85) (end 130.795 86.85) (width 0.25) (layer "F.Cu") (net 13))
 (segment (start 147.4175 68.58) (end 134.37401 68.58) (width 0.25) (layer "F.Cu") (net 13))
 (segment (start 127 86.36) (end 127.49 86.85) (width 0.25) (layer "F.Cu") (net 13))
 (segment (start 134.37401 68.58) (end 127 75.95401) (width 0.25) (layer "F.Cu") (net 13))
 (segment (start 127 75.95401) (end 127 86.36) (width 0.25) (layer "F.Cu") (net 13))
 (segment (start 117.675 78.135) (end 119.38 76.43) (width 0.25) (layer "F.Cu") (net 4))
 (segment (start 138.13 87.135) (end 137 88.265) (width 0.25) (layer "F.Cu") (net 4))
 (segment (start 123.175 89.39) (end 125.715 89.39) (width 0.25) (layer "F.Cu") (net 4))
 (segment (start 125.715 89.39) (end 130.795 94.47) (width 0.25) (layer "F.Cu") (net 4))
 (segment (start 114.3 80.515) (end 123.175 89.39) (width 0.25) (layer "F.Cu") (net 4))
 (segment (start 119.38 76.43) (end 119.38 55.88) (width 0.25) (layer "F.Cu") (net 4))
 (segment (start 124.3 88.265) (end 123.175 89.39) (width 0.25) (layer "F.Cu") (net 4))
 (segment (start 144.915 87.135) (end 138.13 87.135) (width 0.25) (layer "F.Cu") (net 4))
 (segment (start 115.625 78.135) (end 117.675 78.135) (width 0.25) (layer "F.Cu") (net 4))
 (segment (start 119.38 55.88) (end 124.46 50.8) (width 0.25) (layer "F.Cu") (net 4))
 (segment (start 114.3 76.81) (end 114.3 80.515) (width 0.25) (layer "F.Cu") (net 4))
 (segment (start 114.3 76.81) (end 115.625 78.135) (width 0.25) (layer "F.Cu") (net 4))
 (segment (start 114.3 70.51) (end 114.3 76.81) (width 0.25) (layer "F.Cu") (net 4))
 (segment (start 124.46 50.8) (end 124.46 48.385) (width 0.25) (layer "F.Cu") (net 4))
 (segment (start 146.24 88.46) (end 144.915 87.135) (width 0.25) (layer "F.Cu") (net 4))
 (segment (start 137 88.265) (end 124.3 88.265) (width 0.25) (layer "F.Cu") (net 4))
 (segment (start 119.38 101.6) (end 119.38 100.805) (width 0.25) (layer "F.Cu") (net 12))
 (segment (start 119.38 100.805) (end 123.175 97.01) (width 0.25) (layer "F.Cu") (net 12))
 (segment (start 114.2 101.42) (end 114.38 101.6) (width 0.25) (layer "F.Cu") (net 2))
 (segment (start 109.22 101.42) (end 114.2 101.42) (width 0.25) (layer "F.Cu") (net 2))
 (segment (start 109.22 96.52) (end 114.38 96.52) (width 0.25) (layer "F.Cu") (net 1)))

